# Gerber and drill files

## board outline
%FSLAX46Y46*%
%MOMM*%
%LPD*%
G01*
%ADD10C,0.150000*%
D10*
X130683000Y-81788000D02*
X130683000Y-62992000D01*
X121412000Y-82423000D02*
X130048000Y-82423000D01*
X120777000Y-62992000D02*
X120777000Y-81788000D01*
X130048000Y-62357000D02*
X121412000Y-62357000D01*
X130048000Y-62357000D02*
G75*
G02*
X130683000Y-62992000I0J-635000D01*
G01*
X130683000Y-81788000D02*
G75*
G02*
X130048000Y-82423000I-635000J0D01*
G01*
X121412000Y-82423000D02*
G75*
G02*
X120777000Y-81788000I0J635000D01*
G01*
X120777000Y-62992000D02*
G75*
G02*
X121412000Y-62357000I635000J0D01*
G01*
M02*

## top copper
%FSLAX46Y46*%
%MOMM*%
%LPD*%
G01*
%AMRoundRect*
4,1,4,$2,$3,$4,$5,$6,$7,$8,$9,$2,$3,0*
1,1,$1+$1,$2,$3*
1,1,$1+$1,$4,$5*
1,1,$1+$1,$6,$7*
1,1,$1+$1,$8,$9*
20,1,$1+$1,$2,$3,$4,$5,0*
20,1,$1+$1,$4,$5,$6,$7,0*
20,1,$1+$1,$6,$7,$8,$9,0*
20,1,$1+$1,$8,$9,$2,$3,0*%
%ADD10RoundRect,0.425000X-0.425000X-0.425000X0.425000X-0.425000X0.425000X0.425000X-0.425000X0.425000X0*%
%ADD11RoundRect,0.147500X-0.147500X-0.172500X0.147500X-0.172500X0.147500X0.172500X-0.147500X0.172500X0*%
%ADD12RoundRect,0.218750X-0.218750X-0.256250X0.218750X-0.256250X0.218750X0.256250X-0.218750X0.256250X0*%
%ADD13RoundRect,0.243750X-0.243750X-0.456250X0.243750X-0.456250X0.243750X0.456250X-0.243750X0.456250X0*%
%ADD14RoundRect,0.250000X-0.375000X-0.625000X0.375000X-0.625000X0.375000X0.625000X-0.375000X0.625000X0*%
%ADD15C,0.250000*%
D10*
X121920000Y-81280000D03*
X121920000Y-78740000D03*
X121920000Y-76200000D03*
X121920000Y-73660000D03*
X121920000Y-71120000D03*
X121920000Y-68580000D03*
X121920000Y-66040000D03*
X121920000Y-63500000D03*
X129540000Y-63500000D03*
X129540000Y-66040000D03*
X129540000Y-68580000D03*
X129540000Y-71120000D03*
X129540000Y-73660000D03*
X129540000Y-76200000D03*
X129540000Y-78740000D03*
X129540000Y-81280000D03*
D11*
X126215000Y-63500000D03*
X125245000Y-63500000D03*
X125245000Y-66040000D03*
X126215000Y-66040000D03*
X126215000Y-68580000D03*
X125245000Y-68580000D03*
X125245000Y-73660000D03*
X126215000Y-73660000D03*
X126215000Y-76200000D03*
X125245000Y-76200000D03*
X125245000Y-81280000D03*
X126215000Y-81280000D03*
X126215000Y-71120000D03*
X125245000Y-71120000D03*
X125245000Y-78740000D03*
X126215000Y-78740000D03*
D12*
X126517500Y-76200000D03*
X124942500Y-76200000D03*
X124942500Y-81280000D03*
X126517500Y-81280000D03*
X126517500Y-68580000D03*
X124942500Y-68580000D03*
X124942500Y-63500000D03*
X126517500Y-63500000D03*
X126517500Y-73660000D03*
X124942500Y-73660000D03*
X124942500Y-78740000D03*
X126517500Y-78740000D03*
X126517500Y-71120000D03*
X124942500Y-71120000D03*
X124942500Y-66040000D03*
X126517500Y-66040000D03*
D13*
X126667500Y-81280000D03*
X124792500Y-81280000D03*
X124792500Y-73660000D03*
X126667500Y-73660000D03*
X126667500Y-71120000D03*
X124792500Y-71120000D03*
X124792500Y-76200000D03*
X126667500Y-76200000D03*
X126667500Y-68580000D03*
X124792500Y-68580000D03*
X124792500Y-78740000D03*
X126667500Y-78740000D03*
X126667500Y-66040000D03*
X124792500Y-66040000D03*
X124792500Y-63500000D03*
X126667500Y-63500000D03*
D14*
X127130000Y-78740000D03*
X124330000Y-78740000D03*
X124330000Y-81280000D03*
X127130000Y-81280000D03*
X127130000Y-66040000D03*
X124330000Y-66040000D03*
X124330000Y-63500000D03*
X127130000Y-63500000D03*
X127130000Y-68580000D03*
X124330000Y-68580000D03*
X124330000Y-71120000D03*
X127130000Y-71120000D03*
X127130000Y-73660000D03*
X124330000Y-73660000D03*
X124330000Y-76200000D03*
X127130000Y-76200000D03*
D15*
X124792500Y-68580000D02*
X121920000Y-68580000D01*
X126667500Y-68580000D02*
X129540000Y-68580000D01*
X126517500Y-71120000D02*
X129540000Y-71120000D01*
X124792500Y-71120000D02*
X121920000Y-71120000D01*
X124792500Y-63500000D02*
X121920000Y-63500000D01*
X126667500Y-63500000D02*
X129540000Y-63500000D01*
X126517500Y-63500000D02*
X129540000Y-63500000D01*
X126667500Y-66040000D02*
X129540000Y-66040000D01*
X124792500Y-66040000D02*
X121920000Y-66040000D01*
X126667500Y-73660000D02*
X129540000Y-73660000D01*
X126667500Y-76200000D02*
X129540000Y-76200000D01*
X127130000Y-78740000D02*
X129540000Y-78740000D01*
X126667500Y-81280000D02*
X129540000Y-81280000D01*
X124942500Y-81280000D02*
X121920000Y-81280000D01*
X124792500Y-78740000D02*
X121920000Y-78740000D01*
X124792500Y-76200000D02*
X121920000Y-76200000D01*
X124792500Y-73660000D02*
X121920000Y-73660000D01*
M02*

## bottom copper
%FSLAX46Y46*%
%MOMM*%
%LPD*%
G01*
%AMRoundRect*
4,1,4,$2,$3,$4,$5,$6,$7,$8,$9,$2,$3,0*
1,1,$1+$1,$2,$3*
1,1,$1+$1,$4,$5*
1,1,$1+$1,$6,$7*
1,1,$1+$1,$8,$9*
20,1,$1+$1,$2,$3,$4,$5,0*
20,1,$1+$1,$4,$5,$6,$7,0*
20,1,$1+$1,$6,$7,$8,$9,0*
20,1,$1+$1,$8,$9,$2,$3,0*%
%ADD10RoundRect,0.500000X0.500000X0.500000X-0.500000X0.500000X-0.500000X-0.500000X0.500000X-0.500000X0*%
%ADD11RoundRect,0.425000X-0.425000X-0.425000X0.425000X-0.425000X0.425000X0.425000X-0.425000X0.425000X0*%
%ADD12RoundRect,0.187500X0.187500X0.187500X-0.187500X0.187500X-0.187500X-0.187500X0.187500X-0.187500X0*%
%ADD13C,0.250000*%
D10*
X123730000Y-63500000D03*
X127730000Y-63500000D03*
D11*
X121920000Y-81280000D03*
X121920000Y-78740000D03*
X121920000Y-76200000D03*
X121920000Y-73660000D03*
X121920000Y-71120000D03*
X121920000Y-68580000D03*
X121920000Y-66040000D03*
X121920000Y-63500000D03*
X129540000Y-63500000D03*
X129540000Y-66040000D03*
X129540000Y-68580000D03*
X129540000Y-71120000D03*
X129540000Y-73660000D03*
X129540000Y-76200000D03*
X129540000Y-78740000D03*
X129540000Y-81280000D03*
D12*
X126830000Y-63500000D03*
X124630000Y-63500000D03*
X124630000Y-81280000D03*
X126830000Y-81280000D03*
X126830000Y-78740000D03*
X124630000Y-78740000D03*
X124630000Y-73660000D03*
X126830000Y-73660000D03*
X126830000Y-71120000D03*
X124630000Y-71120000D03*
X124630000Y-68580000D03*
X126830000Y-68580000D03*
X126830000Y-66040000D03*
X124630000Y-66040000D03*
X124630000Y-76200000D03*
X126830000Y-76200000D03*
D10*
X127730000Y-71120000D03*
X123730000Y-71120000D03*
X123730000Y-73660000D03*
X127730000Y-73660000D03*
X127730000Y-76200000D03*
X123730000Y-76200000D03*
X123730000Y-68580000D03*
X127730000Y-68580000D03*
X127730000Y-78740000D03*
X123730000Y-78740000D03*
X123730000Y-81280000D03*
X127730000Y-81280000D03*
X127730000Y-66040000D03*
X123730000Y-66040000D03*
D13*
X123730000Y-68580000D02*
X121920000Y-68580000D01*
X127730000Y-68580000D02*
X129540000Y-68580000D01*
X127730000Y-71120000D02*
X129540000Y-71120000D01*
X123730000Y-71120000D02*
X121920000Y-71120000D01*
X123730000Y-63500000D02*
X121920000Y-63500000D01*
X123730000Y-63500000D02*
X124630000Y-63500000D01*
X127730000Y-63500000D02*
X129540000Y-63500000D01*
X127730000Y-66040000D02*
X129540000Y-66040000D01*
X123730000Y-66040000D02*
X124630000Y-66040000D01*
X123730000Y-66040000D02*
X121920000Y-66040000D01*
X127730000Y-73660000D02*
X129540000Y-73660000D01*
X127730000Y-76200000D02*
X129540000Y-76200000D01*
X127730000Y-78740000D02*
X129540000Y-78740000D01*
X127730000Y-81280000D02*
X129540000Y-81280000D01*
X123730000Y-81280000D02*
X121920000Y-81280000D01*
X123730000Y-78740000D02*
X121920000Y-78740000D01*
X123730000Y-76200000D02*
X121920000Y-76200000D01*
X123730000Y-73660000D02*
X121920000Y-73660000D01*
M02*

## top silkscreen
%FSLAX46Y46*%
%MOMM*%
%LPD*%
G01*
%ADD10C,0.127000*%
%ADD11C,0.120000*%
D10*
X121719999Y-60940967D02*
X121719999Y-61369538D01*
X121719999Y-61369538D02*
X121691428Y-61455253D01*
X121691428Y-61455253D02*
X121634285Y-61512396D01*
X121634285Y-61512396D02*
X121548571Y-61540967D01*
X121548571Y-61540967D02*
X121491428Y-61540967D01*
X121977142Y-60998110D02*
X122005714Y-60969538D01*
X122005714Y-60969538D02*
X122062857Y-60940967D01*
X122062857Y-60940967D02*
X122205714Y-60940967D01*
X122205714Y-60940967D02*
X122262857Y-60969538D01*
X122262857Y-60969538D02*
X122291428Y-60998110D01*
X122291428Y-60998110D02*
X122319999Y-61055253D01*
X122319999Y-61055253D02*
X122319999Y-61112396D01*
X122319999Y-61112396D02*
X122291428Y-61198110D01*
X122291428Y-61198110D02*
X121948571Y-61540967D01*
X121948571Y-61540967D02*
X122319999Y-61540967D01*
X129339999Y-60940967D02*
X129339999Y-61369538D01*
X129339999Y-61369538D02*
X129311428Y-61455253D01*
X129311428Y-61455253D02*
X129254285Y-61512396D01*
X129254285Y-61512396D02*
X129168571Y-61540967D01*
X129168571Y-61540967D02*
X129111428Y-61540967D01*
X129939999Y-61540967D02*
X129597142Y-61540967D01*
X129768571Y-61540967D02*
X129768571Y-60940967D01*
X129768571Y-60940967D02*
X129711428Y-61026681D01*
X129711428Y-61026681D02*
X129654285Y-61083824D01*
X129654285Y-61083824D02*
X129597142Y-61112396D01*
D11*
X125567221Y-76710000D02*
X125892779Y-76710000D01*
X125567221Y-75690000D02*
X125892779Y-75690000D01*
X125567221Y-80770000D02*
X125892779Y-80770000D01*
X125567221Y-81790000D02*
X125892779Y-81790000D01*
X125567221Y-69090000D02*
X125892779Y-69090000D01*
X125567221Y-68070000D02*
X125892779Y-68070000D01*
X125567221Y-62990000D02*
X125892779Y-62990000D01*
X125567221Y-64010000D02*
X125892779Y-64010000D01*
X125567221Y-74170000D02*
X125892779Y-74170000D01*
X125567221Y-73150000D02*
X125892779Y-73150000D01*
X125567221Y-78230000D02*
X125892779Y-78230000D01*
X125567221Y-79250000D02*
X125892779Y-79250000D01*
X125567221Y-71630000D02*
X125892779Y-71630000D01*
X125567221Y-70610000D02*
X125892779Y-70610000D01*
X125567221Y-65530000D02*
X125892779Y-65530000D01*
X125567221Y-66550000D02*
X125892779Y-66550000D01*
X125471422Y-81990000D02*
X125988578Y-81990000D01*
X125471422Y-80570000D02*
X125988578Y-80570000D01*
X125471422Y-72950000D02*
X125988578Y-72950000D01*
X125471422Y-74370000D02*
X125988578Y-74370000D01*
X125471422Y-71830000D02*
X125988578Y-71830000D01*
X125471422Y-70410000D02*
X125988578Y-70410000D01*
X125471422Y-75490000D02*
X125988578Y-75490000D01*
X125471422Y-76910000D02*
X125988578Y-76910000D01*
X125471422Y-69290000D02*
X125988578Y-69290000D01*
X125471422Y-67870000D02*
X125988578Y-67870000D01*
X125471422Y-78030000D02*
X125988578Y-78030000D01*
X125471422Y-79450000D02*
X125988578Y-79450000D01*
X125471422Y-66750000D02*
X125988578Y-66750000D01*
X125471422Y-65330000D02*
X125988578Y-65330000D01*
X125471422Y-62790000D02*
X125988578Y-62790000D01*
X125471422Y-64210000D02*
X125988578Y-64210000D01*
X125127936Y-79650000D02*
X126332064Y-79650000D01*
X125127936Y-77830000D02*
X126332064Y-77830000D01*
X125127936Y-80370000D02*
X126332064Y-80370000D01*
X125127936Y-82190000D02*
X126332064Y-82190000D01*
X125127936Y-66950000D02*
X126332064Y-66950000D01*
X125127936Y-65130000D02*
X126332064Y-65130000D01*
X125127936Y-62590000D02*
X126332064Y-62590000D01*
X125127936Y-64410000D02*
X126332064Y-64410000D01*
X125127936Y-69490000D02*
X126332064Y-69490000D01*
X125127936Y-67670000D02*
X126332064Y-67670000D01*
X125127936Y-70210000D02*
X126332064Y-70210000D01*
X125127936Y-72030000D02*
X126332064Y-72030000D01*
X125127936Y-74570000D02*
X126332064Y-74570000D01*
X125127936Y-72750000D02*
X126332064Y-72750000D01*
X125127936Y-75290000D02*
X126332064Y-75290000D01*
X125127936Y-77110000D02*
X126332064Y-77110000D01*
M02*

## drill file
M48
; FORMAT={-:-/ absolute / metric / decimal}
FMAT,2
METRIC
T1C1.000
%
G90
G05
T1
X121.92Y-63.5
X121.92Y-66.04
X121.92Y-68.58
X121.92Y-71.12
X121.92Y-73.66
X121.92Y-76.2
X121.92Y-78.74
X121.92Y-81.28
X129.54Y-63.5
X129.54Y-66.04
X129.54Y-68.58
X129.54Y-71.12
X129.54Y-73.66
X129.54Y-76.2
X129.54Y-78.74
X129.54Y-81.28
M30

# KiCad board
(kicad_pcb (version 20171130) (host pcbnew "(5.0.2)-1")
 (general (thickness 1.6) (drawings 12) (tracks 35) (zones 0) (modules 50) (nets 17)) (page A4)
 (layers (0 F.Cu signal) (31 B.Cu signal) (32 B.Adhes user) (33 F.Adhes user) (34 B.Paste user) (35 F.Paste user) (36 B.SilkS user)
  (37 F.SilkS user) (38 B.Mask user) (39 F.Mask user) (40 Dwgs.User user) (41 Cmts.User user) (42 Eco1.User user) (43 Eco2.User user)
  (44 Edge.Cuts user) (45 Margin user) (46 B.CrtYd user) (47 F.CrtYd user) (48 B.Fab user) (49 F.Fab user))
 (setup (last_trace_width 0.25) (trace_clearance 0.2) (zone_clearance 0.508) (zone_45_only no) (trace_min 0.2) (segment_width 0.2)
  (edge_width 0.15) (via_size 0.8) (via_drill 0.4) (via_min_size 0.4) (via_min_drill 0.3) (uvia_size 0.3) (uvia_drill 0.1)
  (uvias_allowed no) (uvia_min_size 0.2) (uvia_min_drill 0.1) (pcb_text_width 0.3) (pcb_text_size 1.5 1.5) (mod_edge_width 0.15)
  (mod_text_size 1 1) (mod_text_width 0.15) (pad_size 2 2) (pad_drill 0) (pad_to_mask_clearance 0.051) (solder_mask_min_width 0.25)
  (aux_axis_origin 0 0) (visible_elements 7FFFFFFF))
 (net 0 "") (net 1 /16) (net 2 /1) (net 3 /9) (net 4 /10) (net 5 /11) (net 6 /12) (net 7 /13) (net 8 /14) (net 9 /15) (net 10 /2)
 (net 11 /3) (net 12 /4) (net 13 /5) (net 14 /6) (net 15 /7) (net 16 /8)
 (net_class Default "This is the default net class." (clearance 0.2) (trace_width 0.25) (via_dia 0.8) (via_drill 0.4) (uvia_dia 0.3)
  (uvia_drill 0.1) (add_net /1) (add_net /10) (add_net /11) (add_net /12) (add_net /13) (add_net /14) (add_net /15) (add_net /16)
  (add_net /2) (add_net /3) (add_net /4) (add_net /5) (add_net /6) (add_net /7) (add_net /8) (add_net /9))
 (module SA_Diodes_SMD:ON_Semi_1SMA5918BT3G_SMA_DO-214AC (layer B.Cu) (at 125.73 63.5 180)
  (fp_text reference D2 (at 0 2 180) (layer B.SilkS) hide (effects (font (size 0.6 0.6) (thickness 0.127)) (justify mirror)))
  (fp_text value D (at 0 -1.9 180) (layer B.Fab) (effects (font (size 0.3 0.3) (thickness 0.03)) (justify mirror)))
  (pad 2 smd roundrect (at 2 0 180) (size 2 2) (layers B.Cu B.Paste B.Mask) (roundrect_rratio 0.25) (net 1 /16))
  (pad 1 smd roundrect (at -2 0 180) (size 2 2) (layers B.Cu B.Paste B.Mask) (roundrect_rratio 0.25) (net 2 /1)))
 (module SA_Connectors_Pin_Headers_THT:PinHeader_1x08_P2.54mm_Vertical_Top (layer F.Cu) (at 121.92 63.5)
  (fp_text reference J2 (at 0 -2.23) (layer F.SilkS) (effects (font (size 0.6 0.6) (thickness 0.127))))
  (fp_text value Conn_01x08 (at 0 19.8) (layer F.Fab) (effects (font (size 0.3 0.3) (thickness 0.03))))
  (pad 8 thru_hole roundrect (at 0 17.78) (size 1.7 1.7) (drill 1) (layers *.Cu *.Mask) (roundrect_rratio 0.25) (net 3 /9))
  (pad 7 thru_hole roundrect (at 0 15.24) (size 1.7 1.7) (drill 1) (layers *.Cu *.Mask) (roundrect_rratio 0.25) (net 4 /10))
  (pad 6 thru_hole roundrect (at 0 12.7) (size 1.7 1.7) (drill 1) (layers *.Cu *.Mask) (roundrect_rratio 0.25) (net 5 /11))
  (pad 5 thru_hole roundrect (at 0 10.16) (size 1.7 1.7) (drill 1) (layers *.Cu *.Mask) (roundrect_rratio 0.25) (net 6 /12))
  (pad 4 thru_hole roundrect (at 0 7.62) (size 1.7 1.7) (drill 1) (layers *.Cu *.Mask) (roundrect_rratio 0.25) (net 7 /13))
  (pad 3 thru_hole roundrect (at 0 5.08) (size 1.7 1.7) (drill 1) (layers *.Cu *.Mask) (roundrect_rratio 0.25) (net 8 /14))
  (pad 2 thru_hole roundrect (at 0 2.54) (size 1.7 1.7) (drill 1) (layers *.Cu *.Mask) (roundrect_rratio 0.25) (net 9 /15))
  (pad 1 thru_hole roundrect (at 0 0) (size 1.7 1.7) (drill 1) (layers *.Cu *.Mask) (roundrect_rratio 0.25) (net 1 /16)))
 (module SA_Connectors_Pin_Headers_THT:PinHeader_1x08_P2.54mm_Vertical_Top (layer F.Cu) (at 129.54 63.5)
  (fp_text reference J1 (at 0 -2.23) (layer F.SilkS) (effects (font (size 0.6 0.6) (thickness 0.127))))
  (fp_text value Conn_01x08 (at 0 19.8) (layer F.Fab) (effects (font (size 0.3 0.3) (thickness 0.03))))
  (pad 1 thru_hole roundrect (at 0 0) (size 1.7 1.7) (drill 1) (layers *.Cu *.Mask) (roundrect_rratio 0.25) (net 2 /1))
  (pad 2 thru_hole roundrect (at 0 2.54) (size 1.7 1.7) (drill 1) (layers *.Cu *.Mask) (roundrect_rratio 0.25) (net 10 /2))
  (pad 3 thru_hole roundrect (at 0 5.08) (size 1.7 1.7) (drill 1) (layers *.Cu *.Mask) (roundrect_rratio 0.25) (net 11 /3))
  (pad 4 thru_hole roundrect (at 0 7.62) (size 1.7 1.7) (drill 1) (layers *.Cu *.Mask) (roundrect_rratio 0.25) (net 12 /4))
  (pad 5 thru_hole roundrect (at 0 10.16) (size 1.7 1.7) (drill 1) (layers *.Cu *.Mask) (roundrect_rratio 0.25) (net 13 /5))
  (pad 6 thru_hole roundrect (at 0 12.7) (size 1.7 1.7) (drill 1) (layers *.Cu *.Mask) (roundrect_rratio 0.25) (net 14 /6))
  (pad 7 thru_hole roundrect (at 0 15.24) (size 1.7 1.7) (drill 1) (layers *.Cu *.Mask) (roundrect_rratio 0.25) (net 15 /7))
  (pad 8 thru_hole roundrect (at 0 17.78) (size 1.7 1.7) (drill 1) (layers *.Cu *.Mask) (roundrect_rratio 0.25) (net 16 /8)))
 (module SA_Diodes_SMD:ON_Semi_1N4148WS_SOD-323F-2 (layer B.Cu) (at 125.73 63.5 180)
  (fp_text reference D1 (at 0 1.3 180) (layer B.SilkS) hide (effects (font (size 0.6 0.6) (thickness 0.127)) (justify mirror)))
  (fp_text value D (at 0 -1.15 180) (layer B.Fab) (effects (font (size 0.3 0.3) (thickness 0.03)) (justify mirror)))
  (pad 1 smd roundrect (at -1.1 0 180) (size 0.75 0.75) (layers B.Cu B.Paste B.Mask) (roundrect_rratio 0.25) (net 2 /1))
  (pad 2 smd roundrect (at 1.1 0 180) (size 0.75 0.75) (layers B.Cu B.Paste B.Mask) (roundrect_rratio 0.25) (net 1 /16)))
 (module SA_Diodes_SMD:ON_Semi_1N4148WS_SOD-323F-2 (layer B.Cu) (at 125.73 81.28 180)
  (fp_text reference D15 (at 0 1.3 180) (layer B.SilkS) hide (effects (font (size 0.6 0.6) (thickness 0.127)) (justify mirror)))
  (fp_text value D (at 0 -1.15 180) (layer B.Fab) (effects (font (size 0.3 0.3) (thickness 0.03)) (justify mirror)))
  (pad 2 smd roundrect (at 1.1 0 180) (size 0.75 0.75) (layers B.Cu B.Paste B.Mask) (roundrect_rratio 0.25) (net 3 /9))
  (pad 1 smd roundrect (at -1.1 0 180) (size 0.75 0.75) (layers B.Cu B.Paste B.Mask) (roundrect_rratio 0.25) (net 16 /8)))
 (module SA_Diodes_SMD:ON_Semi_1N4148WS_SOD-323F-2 (layer B.Cu) (at 125.73 78.74 180)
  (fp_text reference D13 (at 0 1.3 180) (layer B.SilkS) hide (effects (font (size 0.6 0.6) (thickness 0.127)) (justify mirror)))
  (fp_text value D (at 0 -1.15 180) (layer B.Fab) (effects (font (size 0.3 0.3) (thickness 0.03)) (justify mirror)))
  (pad 1 smd roundrect (at -1.1 0 180) (size 0.75 0.75) (layers B.Cu B.Paste B.Mask) (roundrect_rratio 0.25) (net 15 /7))
  (pad 2 smd roundrect (at 1.1 0 180) (size 0.75 0.75) (layers B.Cu B.Paste B.Mask) (roundrect_rratio 0.25) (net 4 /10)))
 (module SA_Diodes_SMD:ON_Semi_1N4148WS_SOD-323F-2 (layer B.Cu) (at 125.73 73.66 180)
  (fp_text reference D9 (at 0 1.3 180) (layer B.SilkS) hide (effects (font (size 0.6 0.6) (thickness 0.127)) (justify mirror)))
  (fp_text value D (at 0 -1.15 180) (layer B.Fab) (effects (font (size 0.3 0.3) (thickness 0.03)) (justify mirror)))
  (pad 2 smd roundrect (at 1.1 0 180) (size 0.75 0.75) (layers B.Cu B.Paste B.Mask) (roundrect_rratio 0.25) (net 6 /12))
  (pad 1 smd roundrect (at -1.1 0 180) (size 0.75 0.75) (layers B.Cu B.Paste B.Mask) (roundrect_rratio 0.25) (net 13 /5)))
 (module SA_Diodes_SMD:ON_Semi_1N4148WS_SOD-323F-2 (layer B.Cu) (at 125.73 71.12 180)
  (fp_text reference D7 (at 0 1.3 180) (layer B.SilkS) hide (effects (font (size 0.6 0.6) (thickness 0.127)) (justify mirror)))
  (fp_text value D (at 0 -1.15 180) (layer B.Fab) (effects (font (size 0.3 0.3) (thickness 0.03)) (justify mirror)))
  (pad 1 smd roundrect (at -1.1 0 180) (size 0.75 0.75) (layers B.Cu B.Paste B.Mask) (roundrect_rratio 0.25) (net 12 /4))
  (pad 2 smd roundrect (at 1.1 0 180) (size 0.75 0.75) (layers B.Cu B.Paste B.Mask) (roundrect_rratio 0.25) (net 7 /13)))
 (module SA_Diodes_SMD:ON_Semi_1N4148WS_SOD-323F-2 (layer B.Cu) (at 125.73 68.58 180)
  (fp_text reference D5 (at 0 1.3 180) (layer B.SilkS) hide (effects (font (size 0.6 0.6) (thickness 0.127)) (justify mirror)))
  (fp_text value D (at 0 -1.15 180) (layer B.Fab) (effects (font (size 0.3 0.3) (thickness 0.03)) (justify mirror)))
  (pad 2 smd roundrect (at 1.1 0 180) (size 0.75 0.75) (layers B.Cu B.Paste B.Mask) (roundrect_rratio 0.25) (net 8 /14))
  (pad 1 smd roundrect (at -1.1 0 180) (size 0.75 0.75) (layers B.Cu B.Paste B.Mask) (roundrect_rratio 0.25) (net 11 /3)))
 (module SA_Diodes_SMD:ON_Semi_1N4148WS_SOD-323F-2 (layer B.Cu) (at 125.73 66.04 180)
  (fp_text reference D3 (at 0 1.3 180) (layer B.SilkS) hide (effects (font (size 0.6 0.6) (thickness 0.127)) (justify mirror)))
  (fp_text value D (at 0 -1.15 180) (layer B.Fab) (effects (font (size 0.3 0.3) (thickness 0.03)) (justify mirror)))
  (pad 1 smd roundrect (at -1.1 0 180) (size 0.75 0.75) (layers B.Cu B.Paste B.Mask) (roundrect_rratio 0.25) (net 10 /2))
  (pad 2 smd roundrect (at 1.1 0 180) (size 0.75 0.75) (layers B.Cu B.Paste B.Mask) (roundrect_rratio 0.25) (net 9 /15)))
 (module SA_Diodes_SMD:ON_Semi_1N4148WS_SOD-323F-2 (layer B.Cu) (at 125.73 76.2 180)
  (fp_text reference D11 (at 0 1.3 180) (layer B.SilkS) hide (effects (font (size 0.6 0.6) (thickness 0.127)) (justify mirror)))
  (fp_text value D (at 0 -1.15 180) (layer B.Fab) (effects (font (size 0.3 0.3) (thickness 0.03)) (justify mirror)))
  (pad 2 smd roundrect (at 1.1 0 180) (size 0.75 0.75) (layers B.Cu B.Paste B.Mask) (roundrect_rratio 0.25) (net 5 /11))
  (pad 1 smd roundrect (at -1.1 0 180) (size 0.75 0.75) (layers B.Cu B.Paste B.Mask) (roundrect_rratio 0.25) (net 14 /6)))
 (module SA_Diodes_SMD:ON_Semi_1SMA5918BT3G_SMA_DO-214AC (layer B.Cu) (at 125.73 71.12 180)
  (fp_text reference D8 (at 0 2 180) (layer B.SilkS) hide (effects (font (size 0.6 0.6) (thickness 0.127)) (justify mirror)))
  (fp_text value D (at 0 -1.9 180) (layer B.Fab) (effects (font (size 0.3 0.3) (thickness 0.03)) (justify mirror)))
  (pad 1 smd roundrect (at -2 0 180) (size 2 2) (layers B.Cu B.Paste B.Mask) (roundrect_rratio 0.25) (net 12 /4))
  (pad 2 smd roundrect (at 2 0 180) (size 2 2) (layers B.Cu B.Paste B.Mask) (roundrect_rratio 0.25) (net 7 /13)))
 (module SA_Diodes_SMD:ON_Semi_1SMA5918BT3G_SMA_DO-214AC (layer B.Cu) (at 125.73 73.66 180)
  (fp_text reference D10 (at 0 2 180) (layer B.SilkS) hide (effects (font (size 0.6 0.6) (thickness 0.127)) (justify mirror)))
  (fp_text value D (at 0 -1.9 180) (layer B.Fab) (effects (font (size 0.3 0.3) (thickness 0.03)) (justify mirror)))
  (pad 2 smd roundrect (at 2 0 180) (size 2 2) (layers B.Cu B.Paste B.Mask) (roundrect_rratio 0.25) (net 6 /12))
  (pad 1 smd roundrect (at -2 0 180) (size 2 2) (layers B.Cu B.Paste B.Mask) (roundrect_rratio 0.25) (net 13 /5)))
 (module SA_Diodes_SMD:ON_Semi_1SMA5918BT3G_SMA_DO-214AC (layer B.Cu) (at 125.73 76.2 180)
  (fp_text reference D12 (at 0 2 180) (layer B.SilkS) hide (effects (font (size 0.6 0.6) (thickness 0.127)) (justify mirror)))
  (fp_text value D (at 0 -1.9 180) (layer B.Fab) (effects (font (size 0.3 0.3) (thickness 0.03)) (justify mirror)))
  (pad 1 smd roundrect (at -2 0 180) (size 2 2) (layers B.Cu B.Paste B.Mask) (roundrect_rratio 0.25) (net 14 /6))
  (pad 2 smd roundrect (at 2 0 180) (size 2 2) (layers B.Cu B.Paste B.Mask) (roundrect_rratio 0.25) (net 5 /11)))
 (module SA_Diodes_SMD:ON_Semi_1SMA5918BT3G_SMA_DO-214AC (layer B.Cu) (at 125.73 68.58 180)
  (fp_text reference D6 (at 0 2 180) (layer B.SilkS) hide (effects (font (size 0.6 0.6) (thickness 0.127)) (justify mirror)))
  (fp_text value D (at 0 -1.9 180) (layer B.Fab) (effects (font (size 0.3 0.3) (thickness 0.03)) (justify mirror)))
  (pad 2 smd roundrect (at 2 0 180) (size 2 2) (layers B.Cu B.Paste B.Mask) (roundrect_rratio 0.25) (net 8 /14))
  (pad 1 smd roundrect (at -2 0 180) (size 2 2) (layers B.Cu B.Paste B.Mask) (roundrect_rratio 0.25) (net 11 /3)))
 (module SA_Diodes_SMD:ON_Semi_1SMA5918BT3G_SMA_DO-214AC (layer B.Cu) (at 125.73 78.74 180)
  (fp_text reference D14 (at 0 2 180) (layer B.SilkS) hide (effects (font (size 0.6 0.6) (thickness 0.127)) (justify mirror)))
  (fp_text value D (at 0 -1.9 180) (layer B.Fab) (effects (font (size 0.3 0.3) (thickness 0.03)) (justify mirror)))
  (pad 1 smd roundrect (at -2 0 180) (size 2 2) (layers B.Cu B.Paste B.Mask) (roundrect_rratio 0.25) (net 15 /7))
  (pad 2 smd roundrect (at 2 0 180) (size 2 2) (layers B.Cu B.Paste B.Mask) (roundrect_rratio 0.25) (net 4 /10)))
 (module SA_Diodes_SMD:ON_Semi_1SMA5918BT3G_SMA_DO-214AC (layer B.Cu) (at 125.73 81.28 180)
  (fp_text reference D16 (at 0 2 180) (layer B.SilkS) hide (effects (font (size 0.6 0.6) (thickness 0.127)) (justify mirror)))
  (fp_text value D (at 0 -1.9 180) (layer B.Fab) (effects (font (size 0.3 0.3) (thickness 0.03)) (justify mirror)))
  (pad 2 smd roundrect (at 2 0 180) (size 2 2) (layers B.Cu B.Paste B.Mask) (roundrect_rratio 0.25) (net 3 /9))
  (pad 1 smd roundrect (at -2 0 180) (size 2 2) (layers B.Cu B.Paste B.Mask) (roundrect_rratio 0.25) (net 16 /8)))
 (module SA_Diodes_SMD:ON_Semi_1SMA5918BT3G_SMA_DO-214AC (layer B.Cu) (at 125.73 66.04 180)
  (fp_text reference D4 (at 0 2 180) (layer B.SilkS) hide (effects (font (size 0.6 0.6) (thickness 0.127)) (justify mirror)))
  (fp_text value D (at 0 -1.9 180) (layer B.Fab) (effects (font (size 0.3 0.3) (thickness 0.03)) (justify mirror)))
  (pad 1 smd roundrect (at -2 0 180) (size 2 2) (layers B.Cu B.Paste B.Mask) (roundrect_rratio 0.25) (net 10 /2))
  (pad 2 smd roundrect (at 2 0 180) (size 2 2) (layers B.Cu B.Paste B.Mask) (roundrect_rratio 0.25) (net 9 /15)))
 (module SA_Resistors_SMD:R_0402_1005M (layer F.Cu) (at 125.73 63.5)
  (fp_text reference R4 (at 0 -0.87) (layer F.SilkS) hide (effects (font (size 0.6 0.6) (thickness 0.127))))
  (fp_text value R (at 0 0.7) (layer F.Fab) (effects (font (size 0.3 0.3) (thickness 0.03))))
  (pad 2 smd roundrect (at 0.485 0) (size 0.59 0.64) (layers F.Cu F.Paste F.Mask) (roundrect_rratio 0.25) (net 2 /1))
  (pad 1 smd roundrect (at -0.485 0) (size 0.59 0.64) (layers F.Cu F.Paste F.Mask) (roundrect_rratio 0.25) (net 1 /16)))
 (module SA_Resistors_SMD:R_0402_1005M (layer F.Cu) (at 125.73 66.04)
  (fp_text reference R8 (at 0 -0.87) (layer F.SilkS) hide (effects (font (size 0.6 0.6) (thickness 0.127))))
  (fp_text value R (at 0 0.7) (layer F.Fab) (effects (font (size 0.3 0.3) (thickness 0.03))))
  (pad 1 smd roundrect (at -0.485 0) (size 0.59 0.64) (layers F.Cu F.Paste F.Mask) (roundrect_rratio 0.25) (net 9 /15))
  (pad 2 smd roundrect (at 0.485 0) (size 0.59 0.64) (layers F.Cu F.Paste F.Mask) (roundrect_rratio 0.25) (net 10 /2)))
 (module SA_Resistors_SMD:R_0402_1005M (layer F.Cu) (at 125.73 68.58)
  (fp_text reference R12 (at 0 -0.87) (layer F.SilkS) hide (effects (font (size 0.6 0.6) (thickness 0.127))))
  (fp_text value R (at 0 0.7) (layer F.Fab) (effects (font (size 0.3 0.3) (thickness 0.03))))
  (pad 2 smd roundrect (at 0.485 0) (size 0.59 0.64) (layers F.Cu F.Paste F.Mask) (roundrect_rratio 0.25) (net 11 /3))
  (pad 1 smd roundrect (at -0.485 0) (size 0.59 0.64) (layers F.Cu F.Paste F.Mask) (roundrect_rratio 0.25) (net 8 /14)))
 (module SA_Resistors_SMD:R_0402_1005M (layer F.Cu) (at 125.73 73.66)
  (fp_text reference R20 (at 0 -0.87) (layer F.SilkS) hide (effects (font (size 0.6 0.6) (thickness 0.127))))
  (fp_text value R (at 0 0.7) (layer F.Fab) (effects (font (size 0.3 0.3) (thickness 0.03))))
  (pad 1 smd roundrect (at -0.485 0) (size 0.59 0.64) (layers F.Cu F.Paste F.Mask) (roundrect_rratio 0.25) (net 6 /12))
  (pad 2 smd roundrect (at 0.485 0) (size 0.59 0.64) (layers F.Cu F.Paste F.Mask) (roundrect_rratio 0.25) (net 13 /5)))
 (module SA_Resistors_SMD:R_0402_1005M (layer F.Cu) (at 125.73 76.2)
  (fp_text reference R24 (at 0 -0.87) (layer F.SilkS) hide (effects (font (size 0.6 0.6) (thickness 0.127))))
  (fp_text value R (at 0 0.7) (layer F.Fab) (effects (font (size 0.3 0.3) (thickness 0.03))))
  (pad 2 smd roundrect (at 0.485 0) (size 0.59 0.64) (layers F.Cu F.Paste F.Mask) (roundrect_rratio 0.25) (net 14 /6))
  (pad 1 smd roundrect (at -0.485 0) (size 0.59 0.64) (layers F.Cu F.Paste F.Mask) (roundrect_rratio 0.25) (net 5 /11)))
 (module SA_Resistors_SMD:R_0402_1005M (layer F.Cu) (at 125.73 81.28)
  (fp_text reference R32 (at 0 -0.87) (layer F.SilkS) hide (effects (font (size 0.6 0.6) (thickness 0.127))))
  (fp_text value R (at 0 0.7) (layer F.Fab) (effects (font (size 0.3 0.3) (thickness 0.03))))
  (pad 1 smd roundrect (at -0.485 0) (size 0.59 0.64) (layers F.Cu F.Paste F.Mask) (roundrect_rratio 0.25) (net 3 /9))
  (pad 2 smd roundrect (at 0.485 0) (size 0.59 0.64) (layers F.Cu F.Paste F.Mask) (roundrect_rratio 0.25) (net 16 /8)))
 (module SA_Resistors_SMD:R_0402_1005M (layer F.Cu) (at 125.73 71.12)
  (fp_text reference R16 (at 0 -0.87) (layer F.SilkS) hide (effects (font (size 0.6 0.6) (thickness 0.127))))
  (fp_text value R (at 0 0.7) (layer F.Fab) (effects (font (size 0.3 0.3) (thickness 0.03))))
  (pad 2 smd roundrect (at 0.485 0) (size 0.59 0.64) (layers F.Cu F.Paste F.Mask) (roundrect_rratio 0.25) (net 12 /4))
  (pad 1 smd roundrect (at -0.485 0) (size 0.59 0.64) (layers F.Cu F.Paste F.Mask) (roundrect_rratio 0.25) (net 7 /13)))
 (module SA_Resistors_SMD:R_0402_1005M (layer F.Cu) (at 125.73 78.74)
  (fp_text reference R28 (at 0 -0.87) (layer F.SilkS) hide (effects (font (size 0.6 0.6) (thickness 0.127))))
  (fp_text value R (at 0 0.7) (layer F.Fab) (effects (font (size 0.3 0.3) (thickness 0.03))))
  (pad 1 smd roundrect (at -0.485 0) (size 0.59 0.64) (layers F.Cu F.Paste F.Mask) (roundrect_rratio 0.25) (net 4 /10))
  (pad 2 smd roundrect (at 0.485 0) (size 0.59 0.64) (layers F.Cu F.Paste F.Mask) (roundrect_rratio 0.25) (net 15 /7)))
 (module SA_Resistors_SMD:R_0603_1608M (layer F.Cu) (at 125.73 76.2)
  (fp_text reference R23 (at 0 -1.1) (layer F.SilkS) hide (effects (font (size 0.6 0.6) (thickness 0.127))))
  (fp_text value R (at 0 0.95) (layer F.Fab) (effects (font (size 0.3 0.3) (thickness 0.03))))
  (fp_line (start -0.162779 0.51) (end 0.162779 0.51) (layer F.SilkS) (width 0.12))
  (fp_line (start -0.162779 -0.51) (end 0.162779 -0.51) (layer F.SilkS) (width 0.12))
  (pad 2 smd roundrect (at 0.7875 0) (size 0.875 0.95) (layers F.Cu F.Paste F.Mask) (roundrect_rratio 0.25) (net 14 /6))
  (pad 1 smd roundrect (at -0.7875 0) (size 0.875 0.95) (layers F.Cu F.Paste F.Mask) (roundrect_rratio 0.25) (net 5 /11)))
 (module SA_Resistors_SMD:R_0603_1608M (layer F.Cu) (at 125.73 81.28)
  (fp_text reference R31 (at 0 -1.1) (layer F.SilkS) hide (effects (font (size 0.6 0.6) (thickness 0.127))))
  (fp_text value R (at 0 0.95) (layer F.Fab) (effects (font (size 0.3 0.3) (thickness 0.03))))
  (fp_line (start -0.162779 -0.51) (end 0.162779 -0.51) (layer F.SilkS) (width 0.12))
  (fp_line (start -0.162779 0.51) (end 0.162779 0.51) (layer F.SilkS) (width 0.12))
  (pad 1 smd roundrect (at -0.7875 0) (size 0.875 0.95) (layers F.Cu F.Paste F.Mask) (roundrect_rratio 0.25) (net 3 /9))
  (pad 2 smd roundrect (at 0.7875 0) (size 0.875 0.95) (layers F.Cu F.Paste F.Mask) (roundrect_rratio 0.25) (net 16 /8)))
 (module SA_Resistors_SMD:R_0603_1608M (layer F.Cu) (at 125.73 68.58)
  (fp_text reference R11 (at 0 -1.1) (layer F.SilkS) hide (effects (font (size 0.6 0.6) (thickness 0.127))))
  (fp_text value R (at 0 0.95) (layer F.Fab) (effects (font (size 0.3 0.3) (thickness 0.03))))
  (fp_line (start -0.162779 0.51) (end 0.162779 0.51) (layer F.SilkS) (width 0.12))
  (fp_line (start -0.162779 -0.51) (end 0.162779 -0.51) (layer F.SilkS) (width 0.12))
  (pad 2 smd roundrect (at 0.7875 0) (size 0.875 0.95) (layers F.Cu F.Paste F.Mask) (roundrect_rratio 0.25) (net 11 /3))
  (pad 1 smd roundrect (at -0.7875 0) (size 0.875 0.95) (layers F.Cu F.Paste F.Mask) (roundrect_rratio 0.25) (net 8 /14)))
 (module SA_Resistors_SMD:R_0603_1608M (layer F.Cu) (at 125.73 63.5)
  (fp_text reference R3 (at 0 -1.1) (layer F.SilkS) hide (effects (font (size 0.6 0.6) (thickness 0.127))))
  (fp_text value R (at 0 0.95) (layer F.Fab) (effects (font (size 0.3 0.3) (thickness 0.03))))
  (fp_line (start -0.162779 -0.51) (end 0.162779 -0.51) (layer F.SilkS) (width 0.12))
  (fp_line (start -0.162779 0.51) (end 0.162779 0.51) (layer F.SilkS) (width 0.12))
  (pad 1 smd roundrect (at -0.7875 0) (size 0.875 0.95) (layers F.Cu F.Paste F.Mask) (roundrect_rratio 0.25) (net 1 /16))
  (pad 2 smd roundrect (at 0.7875 0) (size 0.875 0.95) (layers F.Cu F.Paste F.Mask) (roundrect_rratio 0.25) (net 2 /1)))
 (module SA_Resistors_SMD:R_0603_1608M (layer F.Cu) (at 125.73 73.66)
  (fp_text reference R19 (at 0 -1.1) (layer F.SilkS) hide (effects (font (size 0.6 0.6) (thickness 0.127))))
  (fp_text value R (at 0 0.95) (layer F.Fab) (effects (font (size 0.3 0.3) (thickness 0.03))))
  (fp_line (start -0.162779 0.51) (end 0.162779 0.51) (layer F.SilkS) (width 0.12))
  (fp_line (start -0.162779 -0.51) (end 0.162779 -0.51) (layer F.SilkS) (width 0.12))
  (pad 2 smd roundrect (at 0.7875 0) (size 0.875 0.95) (layers F.Cu F.Paste F.Mask) (roundrect_rratio 0.25) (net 13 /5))
  (pad 1 smd roundrect (at -0.7875 0) (size 0.875 0.95) (layers F.Cu F.Paste F.Mask) (roundrect_rratio 0.25) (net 6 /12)))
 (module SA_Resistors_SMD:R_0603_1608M (layer F.Cu) (at 125.73 78.74)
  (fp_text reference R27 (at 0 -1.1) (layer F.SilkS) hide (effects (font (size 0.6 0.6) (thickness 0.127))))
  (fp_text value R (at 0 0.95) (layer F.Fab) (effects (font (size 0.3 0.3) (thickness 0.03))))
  (fp_line (start -0.162779 -0.51) (end 0.162779 -0.51) (layer F.SilkS) (width 0.12))
  (fp_line (start -0.162779 0.51) (end 0.162779 0.51) (layer F.SilkS) (width 0.12))
  (pad 1 smd roundrect (at -0.7875 0) (size 0.875 0.95) (layers F.Cu F.Paste F.Mask) (roundrect_rratio 0.25) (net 4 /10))
  (pad 2 smd roundrect (at 0.7875 0) (size 0.875 0.95) (layers F.Cu F.Paste F.Mask) (roundrect_rratio 0.25) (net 15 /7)))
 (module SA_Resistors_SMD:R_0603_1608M (layer F.Cu) (at 125.73 71.12)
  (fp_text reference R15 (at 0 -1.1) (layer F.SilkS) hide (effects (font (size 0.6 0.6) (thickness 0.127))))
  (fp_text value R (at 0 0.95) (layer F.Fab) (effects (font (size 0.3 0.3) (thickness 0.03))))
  (fp_line (start -0.162779 0.51) (end 0.162779 0.51) (layer F.SilkS) (width 0.12))
  (fp_line (start -0.162779 -0.51) (end 0.162779 -0.51) (layer F.SilkS) (width 0.12))
  (pad 2 smd roundrect (at 0.7875 0) (size 0.875 0.95) (layers F.Cu F.Paste F.Mask) (roundrect_rratio 0.25) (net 12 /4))
  (pad 1 smd roundrect (at -0.7875 0) (size 0.875 0.95) (layers F.Cu F.Paste F.Mask) (roundrect_rratio 0.25) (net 7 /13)))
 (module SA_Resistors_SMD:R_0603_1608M (layer F.Cu) (at 125.73 66.04)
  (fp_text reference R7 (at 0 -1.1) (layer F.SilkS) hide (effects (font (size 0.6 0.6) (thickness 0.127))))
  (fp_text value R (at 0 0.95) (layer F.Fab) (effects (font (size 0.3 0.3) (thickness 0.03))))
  (fp_line (start -0.162779 -0.51) (end 0.162779 -0.51) (layer F.SilkS) (width 0.12))
  (fp_line (start -0.162779 0.51) (end 0.162779 0.51) (layer F.SilkS) (width 0.12))
  (pad 1 smd roundrect (at -0.7875 0) (size 0.875 0.95) (layers F.Cu F.Paste F.Mask) (roundrect_rratio 0.25) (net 9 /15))
  (pad 2 smd roundrect (at 0.7875 0) (size 0.875 0.95) (layers F.Cu F.Paste F.Mask) (roundrect_rratio 0.25) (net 10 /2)))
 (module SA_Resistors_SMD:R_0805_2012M (layer F.Cu) (at 125.73 81.28)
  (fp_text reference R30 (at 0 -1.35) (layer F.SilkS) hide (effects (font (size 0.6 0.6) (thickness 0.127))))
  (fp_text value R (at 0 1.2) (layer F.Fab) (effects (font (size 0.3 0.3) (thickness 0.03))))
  (fp_line (start -0.258578 0.71) (end 0.258578 0.71) (layer F.SilkS) (width 0.12))
  (fp_line (start -0.258578 -0.71) (end 0.258578 -0.71) (layer F.SilkS) (width 0.12))
  (pad 2 smd roundrect (at 0.9375 0) (size 0.975 1.4) (layers F.Cu F.Paste F.Mask) (roundrect_rratio 0.25) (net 16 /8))
  (pad 1 smd roundrect (at -0.9375 0) (size 0.975 1.4) (layers F.Cu F.Paste F.Mask) (roundrect_rratio 0.25) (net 3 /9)))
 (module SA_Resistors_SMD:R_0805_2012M (layer F.Cu) (at 125.73 73.66)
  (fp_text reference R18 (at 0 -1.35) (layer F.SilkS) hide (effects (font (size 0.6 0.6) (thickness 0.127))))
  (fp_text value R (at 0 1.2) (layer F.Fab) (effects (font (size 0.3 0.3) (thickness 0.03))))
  (fp_line (start -0.258578 -0.71) (end 0.258578 -0.71) (layer F.SilkS) (width 0.12))
  (fp_line (start -0.258578 0.71) (end 0.258578 0.71) (layer F.SilkS) (width 0.12))
  (pad 1 smd roundrect (at -0.9375 0) (size 0.975 1.4) (layers F.Cu F.Paste F.Mask) (roundrect_rratio 0.25) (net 6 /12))
  (pad 2 smd roundrect (at 0.9375 0) (size 0.975 1.4) (layers F.Cu F.Paste F.Mask) (roundrect_rratio 0.25) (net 13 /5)))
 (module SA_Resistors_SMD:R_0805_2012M (layer F.Cu) (at 125.73 71.12)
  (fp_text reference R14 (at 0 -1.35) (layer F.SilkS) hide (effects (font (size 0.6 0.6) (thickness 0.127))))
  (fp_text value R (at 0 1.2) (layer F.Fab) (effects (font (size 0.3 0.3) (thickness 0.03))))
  (fp_line (start -0.258578 0.71) (end 0.258578 0.71) (layer F.SilkS) (width 0.12))
  (fp_line (start -0.258578 -0.71) (end 0.258578 -0.71) (layer F.SilkS) (width 0.12))
  (pad 2 smd roundrect (at 0.9375 0) (size 0.975 1.4) (layers F.Cu F.Paste F.Mask) (roundrect_rratio 0.25) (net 12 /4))
  (pad 1 smd roundrect (at -0.9375 0) (size 0.975 1.4) (layers F.Cu F.Paste F.Mask) (roundrect_rratio 0.25) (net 7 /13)))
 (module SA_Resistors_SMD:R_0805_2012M (layer F.Cu) (at 125.73 76.2)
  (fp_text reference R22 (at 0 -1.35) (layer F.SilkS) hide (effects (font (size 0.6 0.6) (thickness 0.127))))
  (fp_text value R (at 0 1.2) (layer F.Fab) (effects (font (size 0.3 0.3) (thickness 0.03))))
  (fp_line (start -0.258578 -0.71) (end 0.258578 -0.71) (layer F.SilkS) (width 0.12))
  (fp_line (start -0.258578 0.71) (end 0.258578 0.71) (layer F.SilkS) (width 0.12))
  (pad 1 smd roundrect (at -0.9375 0) (size 0.975 1.4) (layers F.Cu F.Paste F.Mask) (roundrect_rratio 0.25) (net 5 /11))
  (pad 2 smd roundrect (at 0.9375 0) (size 0.975 1.4) (layers F.Cu F.Paste F.Mask) (roundrect_rratio 0.25) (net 14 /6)))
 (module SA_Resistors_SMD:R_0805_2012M (layer F.Cu) (at 125.73 68.58)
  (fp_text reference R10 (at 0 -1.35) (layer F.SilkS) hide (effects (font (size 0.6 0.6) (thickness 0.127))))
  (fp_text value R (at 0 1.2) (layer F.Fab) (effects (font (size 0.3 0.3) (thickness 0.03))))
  (fp_line (start -0.258578 0.71) (end 0.258578 0.71) (layer F.SilkS) (width 0.12))
  (fp_line (start -0.258578 -0.71) (end 0.258578 -0.71) (layer F.SilkS) (width 0.12))
  (pad 2 smd roundrect (at 0.9375 0) (size 0.975 1.4) (layers F.Cu F.Paste F.Mask) (roundrect_rratio 0.25) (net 11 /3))
  (pad 1 smd roundrect (at -0.9375 0) (size 0.975 1.4) (layers F.Cu F.Paste F.Mask) (roundrect_rratio 0.25) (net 8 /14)))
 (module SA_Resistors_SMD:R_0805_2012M (layer F.Cu) (at 125.73 78.74)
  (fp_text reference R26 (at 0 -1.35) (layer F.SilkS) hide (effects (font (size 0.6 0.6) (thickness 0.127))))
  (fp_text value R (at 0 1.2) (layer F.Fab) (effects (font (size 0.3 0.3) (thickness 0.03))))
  (fp_line (start -0.258578 -0.71) (end 0.258578 -0.71) (layer F.SilkS) (width 0.12))
  (fp_line (start -0.258578 0.71) (end 0.258578 0.71) (layer F.SilkS) (width 0.12))
  (pad 1 smd roundrect (at -0.9375 0) (size 0.975 1.4) (layers F.Cu F.Paste F.Mask) (roundrect_rratio 0.25) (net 4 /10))
  (pad 2 smd roundrect (at 0.9375 0) (size 0.975 1.4) (layers F.Cu F.Paste F.Mask) (roundrect_rratio 0.25) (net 15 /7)))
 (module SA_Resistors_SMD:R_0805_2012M (layer F.Cu) (at 125.73 66.04)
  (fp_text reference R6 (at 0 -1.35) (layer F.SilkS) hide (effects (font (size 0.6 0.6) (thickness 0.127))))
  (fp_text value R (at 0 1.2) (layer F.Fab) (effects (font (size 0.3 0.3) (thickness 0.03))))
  (fp_line (start -0.258578 0.71) (end 0.258578 0.71) (layer F.SilkS) (width 0.12))
  (fp_line (start -0.258578 -0.71) (end 0.258578 -0.71) (layer F.SilkS) (width 0.12))
  (pad 2 smd roundrect (at 0.9375 0) (size 0.975 1.4) (layers F.Cu F.Paste F.Mask) (roundrect_rratio 0.25) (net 10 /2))
  (pad 1 smd roundrect (at -0.9375 0) (size 0.975 1.4) (layers F.Cu F.Paste F.Mask) (roundrect_rratio 0.25) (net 9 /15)))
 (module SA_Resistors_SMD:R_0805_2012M (layer F.Cu) (at 125.73 63.5)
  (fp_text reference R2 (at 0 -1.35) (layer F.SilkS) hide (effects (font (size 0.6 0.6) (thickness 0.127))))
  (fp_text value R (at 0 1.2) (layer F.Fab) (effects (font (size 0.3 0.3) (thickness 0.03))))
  (fp_line (start -0.258578 -0.71) (end 0.258578 -0.71) (layer F.SilkS) (width 0.12))
  (fp_line (start -0.258578 0.71) (end 0.258578 0.71) (layer F.SilkS) (width 0.12))
  (pad 1 smd roundrect (at -0.9375 0) (size 0.975 1.4) (layers F.Cu F.Paste F.Mask) (roundrect_rratio 0.25) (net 1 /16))
  (pad 2 smd roundrect (at 0.9375 0) (size 0.975 1.4) (layers F.Cu F.Paste F.Mask) (roundrect_rratio 0.25) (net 2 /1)))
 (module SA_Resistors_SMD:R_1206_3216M (layer F.Cu) (at 125.73 78.74)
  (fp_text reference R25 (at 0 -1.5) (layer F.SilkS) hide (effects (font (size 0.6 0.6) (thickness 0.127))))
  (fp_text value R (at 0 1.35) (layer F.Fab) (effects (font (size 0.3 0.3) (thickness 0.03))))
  (fp_line (start -0.602064 0.91) (end 0.602064 0.91) (layer F.SilkS) (width 0.12))
  (fp_line (start -0.602064 -0.91) (end 0.602064 -0.91) (layer F.SilkS) (width 0.12))
  (pad 2 smd roundrect (at 1.4 0) (size 1.25 1.75) (layers F.Cu F.Paste F.Mask) (roundrect_rratio 0.2) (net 15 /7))
  (pad 1 smd roundrect (at -1.4 0) (size 1.25 1.75) (layers F.Cu F.Paste F.Mask) (roundrect_rratio 0.2) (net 4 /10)))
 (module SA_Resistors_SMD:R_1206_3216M (layer F.Cu) (at 125.73 81.28)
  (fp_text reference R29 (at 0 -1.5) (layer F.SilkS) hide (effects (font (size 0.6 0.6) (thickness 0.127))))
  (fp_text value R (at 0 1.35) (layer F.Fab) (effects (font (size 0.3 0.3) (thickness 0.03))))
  (fp_line (start -0.602064 -0.91) (end 0.602064 -0.91) (layer F.SilkS) (width 0.12))
  (fp_line (start -0.602064 0.91) (end 0.602064 0.91) (layer F.SilkS) (width 0.12))
  (pad 1 smd roundrect (at -1.4 0) (size 1.25 1.75) (layers F.Cu F.Paste F.Mask) (roundrect_rratio 0.2) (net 3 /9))
  (pad 2 smd roundrect (at 1.4 0) (size 1.25 1.75) (layers F.Cu F.Paste F.Mask) (roundrect_rratio 0.2) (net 16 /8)))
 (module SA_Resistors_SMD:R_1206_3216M (layer F.Cu) (at 125.73 66.04)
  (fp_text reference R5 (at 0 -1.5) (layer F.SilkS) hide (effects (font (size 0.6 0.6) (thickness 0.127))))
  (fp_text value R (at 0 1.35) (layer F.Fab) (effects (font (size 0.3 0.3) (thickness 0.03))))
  (fp_line (start -0.602064 0.91) (end 0.602064 0.91) (layer F.SilkS) (width 0.12))
  (fp_line (start -0.602064 -0.91) (end 0.602064 -0.91) (layer F.SilkS) (width 0.12))
  (pad 2 smd roundrect (at 1.4 0) (size 1.25 1.75) (layers F.Cu F.Paste F.Mask) (roundrect_rratio 0.2) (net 10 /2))
  (pad 1 smd roundrect (at -1.4 0) (size 1.25 1.75) (layers F.Cu F.Paste F.Mask) (roundrect_rratio 0.2) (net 9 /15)))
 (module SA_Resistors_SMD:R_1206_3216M (layer F.Cu) (at 125.73 63.5)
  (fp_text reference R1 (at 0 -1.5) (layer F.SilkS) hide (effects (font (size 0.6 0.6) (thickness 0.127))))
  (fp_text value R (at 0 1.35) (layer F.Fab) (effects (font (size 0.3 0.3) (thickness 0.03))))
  (fp_line (start -0.602064 -0.91) (end 0.602064 -0.91) (layer F.SilkS) (width 0.12))
  (fp_line (start -0.602064 0.91) (end 0.602064 0.91) (layer F.SilkS) (width 0.12))
  (pad 1 smd roundrect (at -1.4 0) (size 1.25 1.75) (layers F.Cu F.Paste F.Mask) (roundrect_rratio 0.2) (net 1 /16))
  (pad 2 smd roundrect (at 1.4 0) (size 1.25 1.75) (layers F.Cu F.Paste F.Mask) (roundrect_rratio 0.2) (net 2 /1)))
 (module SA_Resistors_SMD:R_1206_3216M (layer F.Cu) (at 125.73 68.58)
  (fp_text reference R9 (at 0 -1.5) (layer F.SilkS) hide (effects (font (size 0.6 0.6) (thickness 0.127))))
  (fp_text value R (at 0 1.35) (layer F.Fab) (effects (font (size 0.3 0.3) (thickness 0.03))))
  (fp_line (start -0.602064 0.91) (end 0.602064 0.91) (layer F.SilkS) (width 0.12))
  (fp_line (start -0.602064 -0.91) (end 0.602064 -0.91) (layer F.SilkS) (width 0.12))
  (pad 2 smd roundrect (at 1.4 0) (size 1.25 1.75) (layers F.Cu F.Paste F.Mask) (roundrect_rratio 0.2) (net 11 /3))
  (pad 1 smd roundrect (at -1.4 0) (size 1.25 1.75) (layers F.Cu F.Paste F.Mask) (roundrect_rratio 0.2) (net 8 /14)))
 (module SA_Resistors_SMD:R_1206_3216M (layer F.Cu) (at 125.73 71.12)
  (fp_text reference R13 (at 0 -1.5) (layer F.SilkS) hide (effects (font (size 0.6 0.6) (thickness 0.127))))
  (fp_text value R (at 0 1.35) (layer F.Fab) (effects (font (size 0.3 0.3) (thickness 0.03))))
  (fp_line (start -0.602064 -0.91) (end 0.602064 -0.91) (layer F.SilkS) (width 0.12))
  (fp_line (start -0.602064 0.91) (end 0.602064 0.91) (layer F.SilkS) (width 0.12))
  (pad 1 smd roundrect (at -1.4 0) (size 1.25 1.75) (layers F.Cu F.Paste F.Mask) (roundrect_rratio 0.2) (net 7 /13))
  (pad 2 smd roundrect (at 1.4 0) (size 1.25 1.75) (layers F.Cu F.Paste F.Mask) (roundrect_rratio 0.2) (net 12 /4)))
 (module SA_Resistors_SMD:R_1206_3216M (layer F.Cu) (at 125.73 73.66)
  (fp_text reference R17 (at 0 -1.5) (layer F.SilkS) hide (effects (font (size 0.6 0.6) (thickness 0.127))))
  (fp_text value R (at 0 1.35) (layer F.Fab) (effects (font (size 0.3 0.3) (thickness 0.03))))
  (fp_line (start -0.602064 0.91) (end 0.602064 0.91) (layer F.SilkS) (width 0.12))
  (fp_line (start -0.602064 -0.91) (end 0.602064 -0.91) (layer F.SilkS) (width 0.12))
  (pad 2 smd roundrect (at 1.4 0) (size 1.25 1.75) (layers F.Cu F.Paste F.Mask) (roundrect_rratio 0.2) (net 13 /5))
  (pad 1 smd roundrect (at -1.4 0) (size 1.25 1.75) (layers F.Cu F.Paste F.Mask) (roundrect_rratio 0.2) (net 6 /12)))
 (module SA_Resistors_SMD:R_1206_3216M (layer F.Cu) (at 125.73 76.2)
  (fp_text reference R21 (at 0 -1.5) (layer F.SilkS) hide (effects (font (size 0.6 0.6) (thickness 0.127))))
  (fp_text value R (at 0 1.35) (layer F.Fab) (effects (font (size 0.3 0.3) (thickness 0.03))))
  (fp_line (start -0.602064 -0.91) (end 0.602064 -0.91) (layer F.SilkS) (width 0.12))
  (fp_line (start -0.602064 0.91) (end 0.602064 0.91) (layer F.SilkS) (width 0.12))
  (pad 1 smd roundrect (at -1.4 0) (size 1.25 1.75) (layers F.Cu F.Paste F.Mask) (roundrect_rratio 0.2) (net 5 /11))
  (pad 2 smd roundrect (at 1.4 0) (size 1.25 1.75) (layers F.Cu F.Paste F.Mask) (roundrect_rratio 0.2) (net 14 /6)))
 (gr_line (start 130.683 81.788) (end 130.683 62.992) (layer Edge.Cuts) (width 0.15))
 (gr_line (start 121.412 82.423) (end 130.048 82.423) (layer Edge.Cuts) (width 0.15))
 (gr_line (start 120.777 62.992) (end 120.777 81.788) (layer Edge.Cuts) (width 0.15))
 (gr_line (start 130.048 62.357) (end 121.412 62.357) (layer Edge.Cuts) (width 0.15))
 (gr_arc (start 130.048 62.992) (end 130.683 62.992) (angle -90) (layer Edge.Cuts) (width 0.15))
 (gr_arc (start 130.048 81.788) (end 130.048 82.423) (angle -90) (layer Edge.Cuts) (width 0.15))
 (gr_arc (start 121.412 81.788) (end 120.777 81.788) (angle -90) (layer Edge.Cuts) (width 0.15))
 (gr_arc (start 121.412 62.992) (end 121.412 62.357) (angle -90) (layer Edge.Cuts) (width 0.15))
 (segment (start 124.7925 68.58) (end 121.92 68.58) (width 0.25) (layer F.Cu) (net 8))
 (segment (start 123.73 68.58) (end 121.92 68.58) (width 0.25) (layer B.Cu) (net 8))
 (segment (start 126.6675 68.58) (end 129.54 68.58) (width 0.25) (layer F.Cu) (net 11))
 (segment (start 127.73 68.58) (end 129.54 68.58) (width 0.25) (layer B.Cu) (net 11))
 (segment (start 126.5175 71.12) (end 129.54 71.12) (width 0.25) (layer F.Cu) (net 12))
 (segment (start 127.73 71.12) (end 129.54 71.12) (width 0.25) (layer B.Cu) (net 12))
 (segment (start 124.7925 71.12) (end 121.92 71.12) (width 0.25) (layer F.Cu) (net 7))
 (segment (start 123.73 71.12) (end 121.92 71.12) (width 0.25) (layer B.Cu) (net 7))
 (segment (start 124.7925 63.5) (end 121.92 63.5) (width 0.25) (layer F.Cu) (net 1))
 (segment (start 123.73 63.5) (end 121.92 63.5) (width 0.25) (layer B.Cu) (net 1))
 (segment (start 123.73 63.5) (end 124.63 63.5) (width 0.25) (layer B.Cu) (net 1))
 (segment (start 126.6675 63.5) (end 129.54 63.5) (width 0.25) (layer F.Cu) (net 2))
 (segment (start 126.5175 63.5) (end 129.54 63.5) (width 0.25) (layer F.Cu) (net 2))
 (segment (start 127.73 63.5) (end 129.54 63.5) (width 0.25) (layer B.Cu) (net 2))
 (segment (start 126.6675 66.04) (end 129.54 66.04) (width 0.25) (layer F.Cu) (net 10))
 (segment (start 127.73 66.04) (end 129.54 66.04) (width 0.25) (layer B.Cu) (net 10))
 (segment (start 124.7925 66.04) (end 121.92 66.04) (width 0.25) (layer F.Cu) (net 9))
 (segment (start 123.73 66.04) (end 124.63 66.04) (width 0.25) (layer B.Cu) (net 9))
 (segment (start 123.73 66.04) (end 121.92 66.04) (width 0.25) (layer B.Cu) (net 9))
 (segment (start 126.6675 73.66) (end 129.54 73.66) (width 0.25) (layer F.Cu) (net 13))
 (segment (start 127.73 73.66) (end 129.54 73.66) (width 0.25) (layer B.Cu) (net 13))
 (segment (start 126.6675 76.2) (end 129.54 76.2) (width 0.25) (layer F.Cu) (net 14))
 (segment (start 127.73 76.2) (end 129.54 76.2) (width 0.25) (layer B.Cu) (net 14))
 (segment (start 127.13 78.74) (end 129.54 78.74) (width 0.25) (layer F.Cu) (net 15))
 (segment (start 127.73 78.74) (end 129.54 78.74) (width 0.25) (layer B.Cu) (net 15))
 (segment (start 126.6675 81.28) (end 129.54 81.28) (width 0.25) (layer F.Cu) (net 16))
 (segment (start 127.73 81.28) (end 129.54 81.28) (width 0.25) (layer B.Cu) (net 16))
 (segment (start 124.9425 81.28) (end 121.92 81.28) (width 0.25) (layer F.Cu) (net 3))
 (segment (start 123.73 81.28) (end 121.92 81.28) (width 0.25) (layer B.Cu) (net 3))
 (segment (start 124.7925 78.74) (end 121.92 78.74) (width 0.25) (layer F.Cu) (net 4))
 (segment (start 123.73 78.74) (end 121.92 78.74) (width 0.25) (layer B.Cu) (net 4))
 (segment (start 124.7925 76.2) (end 121.92 76.2) (width 0.25) (layer F.Cu) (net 5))
 (segment (start 123.73 76.2) (end 121.92 76.2) (width 0.25) (layer B.Cu) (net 5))
 (segment (start 124.7925 73.66) (end 121.92 73.66) (width 0.25) (layer F.Cu) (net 6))
 (segment (start 123.73 73.66) (end 121.92 73.66) (width 0.25) (layer B.Cu) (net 6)))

